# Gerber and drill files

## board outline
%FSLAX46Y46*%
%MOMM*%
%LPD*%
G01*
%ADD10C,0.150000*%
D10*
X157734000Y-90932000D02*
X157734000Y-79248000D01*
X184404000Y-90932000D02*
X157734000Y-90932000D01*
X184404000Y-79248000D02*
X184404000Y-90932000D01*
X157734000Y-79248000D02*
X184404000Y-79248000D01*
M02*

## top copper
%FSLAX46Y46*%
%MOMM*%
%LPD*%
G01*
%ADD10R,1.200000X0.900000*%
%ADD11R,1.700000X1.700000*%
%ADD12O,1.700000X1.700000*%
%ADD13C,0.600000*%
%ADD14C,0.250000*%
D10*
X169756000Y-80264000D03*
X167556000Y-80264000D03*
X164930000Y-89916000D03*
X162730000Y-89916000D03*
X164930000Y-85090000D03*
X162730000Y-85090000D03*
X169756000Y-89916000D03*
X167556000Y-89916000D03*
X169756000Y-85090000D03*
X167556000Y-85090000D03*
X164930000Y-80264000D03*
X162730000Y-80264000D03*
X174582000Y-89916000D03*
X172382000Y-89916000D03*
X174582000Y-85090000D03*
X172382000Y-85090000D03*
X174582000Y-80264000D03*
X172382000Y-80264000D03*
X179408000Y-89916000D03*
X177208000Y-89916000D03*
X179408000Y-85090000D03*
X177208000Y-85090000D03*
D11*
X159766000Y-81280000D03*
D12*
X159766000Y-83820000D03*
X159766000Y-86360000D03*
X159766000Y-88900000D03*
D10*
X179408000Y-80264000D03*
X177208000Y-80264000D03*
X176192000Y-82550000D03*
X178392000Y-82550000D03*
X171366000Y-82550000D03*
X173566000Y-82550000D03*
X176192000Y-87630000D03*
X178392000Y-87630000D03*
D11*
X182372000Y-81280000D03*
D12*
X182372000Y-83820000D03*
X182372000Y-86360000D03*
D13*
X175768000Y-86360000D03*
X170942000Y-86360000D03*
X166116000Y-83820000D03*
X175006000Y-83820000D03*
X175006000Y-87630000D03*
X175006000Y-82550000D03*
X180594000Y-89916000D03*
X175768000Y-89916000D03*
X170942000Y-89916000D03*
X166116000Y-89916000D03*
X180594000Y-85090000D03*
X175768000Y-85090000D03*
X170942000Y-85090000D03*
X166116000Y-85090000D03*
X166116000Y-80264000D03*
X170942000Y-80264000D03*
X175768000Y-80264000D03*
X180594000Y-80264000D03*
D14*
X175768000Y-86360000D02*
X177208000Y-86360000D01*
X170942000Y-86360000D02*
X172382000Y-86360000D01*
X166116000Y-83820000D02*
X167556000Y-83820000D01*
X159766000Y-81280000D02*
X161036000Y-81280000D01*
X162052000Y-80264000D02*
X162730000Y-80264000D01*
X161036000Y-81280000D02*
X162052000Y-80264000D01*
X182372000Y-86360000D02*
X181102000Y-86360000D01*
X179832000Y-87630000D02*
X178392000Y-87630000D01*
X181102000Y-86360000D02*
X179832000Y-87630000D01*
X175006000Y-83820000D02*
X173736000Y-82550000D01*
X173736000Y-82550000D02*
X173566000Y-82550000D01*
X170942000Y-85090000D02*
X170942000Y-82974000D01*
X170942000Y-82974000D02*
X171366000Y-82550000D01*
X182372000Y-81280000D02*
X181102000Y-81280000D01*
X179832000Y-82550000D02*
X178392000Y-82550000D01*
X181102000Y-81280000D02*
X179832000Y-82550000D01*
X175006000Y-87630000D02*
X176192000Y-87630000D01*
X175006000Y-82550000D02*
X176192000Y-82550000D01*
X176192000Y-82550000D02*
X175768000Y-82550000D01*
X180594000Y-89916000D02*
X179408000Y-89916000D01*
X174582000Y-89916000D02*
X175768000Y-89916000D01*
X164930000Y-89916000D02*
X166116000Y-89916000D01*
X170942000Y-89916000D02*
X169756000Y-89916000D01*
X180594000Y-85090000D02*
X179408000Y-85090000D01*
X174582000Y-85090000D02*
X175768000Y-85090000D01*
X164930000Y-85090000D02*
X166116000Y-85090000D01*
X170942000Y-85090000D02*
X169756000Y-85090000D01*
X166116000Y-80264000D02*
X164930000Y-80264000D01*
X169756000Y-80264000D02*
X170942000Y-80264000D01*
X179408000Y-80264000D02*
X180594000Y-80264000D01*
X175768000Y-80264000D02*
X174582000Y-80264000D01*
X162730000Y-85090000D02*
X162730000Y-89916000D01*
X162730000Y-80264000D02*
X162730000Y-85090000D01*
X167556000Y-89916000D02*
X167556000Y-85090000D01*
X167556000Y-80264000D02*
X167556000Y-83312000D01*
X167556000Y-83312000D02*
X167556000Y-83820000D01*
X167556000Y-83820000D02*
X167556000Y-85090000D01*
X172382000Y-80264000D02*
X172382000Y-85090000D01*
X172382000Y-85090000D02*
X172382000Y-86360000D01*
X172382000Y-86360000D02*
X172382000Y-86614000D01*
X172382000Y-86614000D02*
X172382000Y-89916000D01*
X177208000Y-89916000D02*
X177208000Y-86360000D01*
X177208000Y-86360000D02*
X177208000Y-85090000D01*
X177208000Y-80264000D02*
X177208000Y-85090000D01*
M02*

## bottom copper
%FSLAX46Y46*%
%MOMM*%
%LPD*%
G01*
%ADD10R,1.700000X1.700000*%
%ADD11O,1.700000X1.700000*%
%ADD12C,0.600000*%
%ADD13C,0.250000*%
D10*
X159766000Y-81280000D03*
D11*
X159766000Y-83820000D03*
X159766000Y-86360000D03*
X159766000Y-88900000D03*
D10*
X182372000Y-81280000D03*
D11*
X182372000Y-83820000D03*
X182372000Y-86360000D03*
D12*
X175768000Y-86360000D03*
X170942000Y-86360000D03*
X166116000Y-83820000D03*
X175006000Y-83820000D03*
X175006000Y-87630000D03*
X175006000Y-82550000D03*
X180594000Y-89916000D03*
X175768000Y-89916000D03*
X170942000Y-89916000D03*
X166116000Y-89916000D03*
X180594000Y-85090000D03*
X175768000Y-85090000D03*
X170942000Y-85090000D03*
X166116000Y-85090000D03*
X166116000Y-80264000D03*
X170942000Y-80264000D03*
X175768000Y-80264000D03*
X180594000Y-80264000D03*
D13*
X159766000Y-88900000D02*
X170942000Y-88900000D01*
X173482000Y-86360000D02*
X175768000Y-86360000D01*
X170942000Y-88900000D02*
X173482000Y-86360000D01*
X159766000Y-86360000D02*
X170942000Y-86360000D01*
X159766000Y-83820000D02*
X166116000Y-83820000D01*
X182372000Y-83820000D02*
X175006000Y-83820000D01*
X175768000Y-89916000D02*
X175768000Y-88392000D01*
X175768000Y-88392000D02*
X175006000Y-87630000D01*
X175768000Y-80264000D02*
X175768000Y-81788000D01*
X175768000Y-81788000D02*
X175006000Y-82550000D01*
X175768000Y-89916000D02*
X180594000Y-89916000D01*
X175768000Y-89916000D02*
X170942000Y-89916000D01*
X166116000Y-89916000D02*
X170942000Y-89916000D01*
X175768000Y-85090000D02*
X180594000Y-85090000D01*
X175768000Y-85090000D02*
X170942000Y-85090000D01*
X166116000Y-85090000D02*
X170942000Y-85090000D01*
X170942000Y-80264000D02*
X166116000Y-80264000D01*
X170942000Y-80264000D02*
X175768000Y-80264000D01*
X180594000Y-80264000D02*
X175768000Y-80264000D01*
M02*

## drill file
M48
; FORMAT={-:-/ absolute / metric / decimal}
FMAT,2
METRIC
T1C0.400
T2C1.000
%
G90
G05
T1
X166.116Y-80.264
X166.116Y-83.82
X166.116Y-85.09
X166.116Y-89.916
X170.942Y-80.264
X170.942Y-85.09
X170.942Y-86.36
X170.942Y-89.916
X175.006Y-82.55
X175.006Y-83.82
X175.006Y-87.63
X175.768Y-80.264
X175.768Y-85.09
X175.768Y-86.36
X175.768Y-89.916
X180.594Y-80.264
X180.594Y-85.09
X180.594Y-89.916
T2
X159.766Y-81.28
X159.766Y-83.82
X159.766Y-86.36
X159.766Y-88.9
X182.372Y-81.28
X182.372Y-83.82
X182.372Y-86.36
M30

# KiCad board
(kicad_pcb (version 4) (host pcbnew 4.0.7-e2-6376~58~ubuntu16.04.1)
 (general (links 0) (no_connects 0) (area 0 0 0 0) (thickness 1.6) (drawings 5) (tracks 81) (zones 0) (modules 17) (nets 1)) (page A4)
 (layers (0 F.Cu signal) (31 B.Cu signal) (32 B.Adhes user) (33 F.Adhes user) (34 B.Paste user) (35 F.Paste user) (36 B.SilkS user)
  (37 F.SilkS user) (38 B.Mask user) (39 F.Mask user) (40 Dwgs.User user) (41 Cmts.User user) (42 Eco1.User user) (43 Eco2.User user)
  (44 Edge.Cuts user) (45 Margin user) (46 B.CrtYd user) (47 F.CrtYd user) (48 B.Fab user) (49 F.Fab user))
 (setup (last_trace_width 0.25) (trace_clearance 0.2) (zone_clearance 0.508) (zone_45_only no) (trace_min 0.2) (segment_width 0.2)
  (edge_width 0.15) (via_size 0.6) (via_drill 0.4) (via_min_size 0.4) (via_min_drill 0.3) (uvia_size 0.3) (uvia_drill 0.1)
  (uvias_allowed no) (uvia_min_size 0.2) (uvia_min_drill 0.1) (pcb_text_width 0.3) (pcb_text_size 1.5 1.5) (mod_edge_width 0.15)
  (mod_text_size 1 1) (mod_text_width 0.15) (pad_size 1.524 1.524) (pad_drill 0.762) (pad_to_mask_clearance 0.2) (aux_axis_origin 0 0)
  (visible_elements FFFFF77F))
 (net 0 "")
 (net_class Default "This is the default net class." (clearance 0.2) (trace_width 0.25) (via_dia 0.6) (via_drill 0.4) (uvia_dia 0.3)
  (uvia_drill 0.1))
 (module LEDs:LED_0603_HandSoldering (layer F.Cu) (at 168.656 80.264 180)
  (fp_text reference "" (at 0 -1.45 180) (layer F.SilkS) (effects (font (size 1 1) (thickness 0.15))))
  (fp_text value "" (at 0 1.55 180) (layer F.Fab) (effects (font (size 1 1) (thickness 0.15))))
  (pad 1 smd rect (at -1.1 0 180) (size 1.2 0.9) (layers F.Cu F.Paste F.Mask))
  (pad 2 smd rect (at 1.1 0 180) (size 1.2 0.9) (layers F.Cu F.Paste F.Mask)))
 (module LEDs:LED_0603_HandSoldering (layer F.Cu) (at 163.83 89.916 180)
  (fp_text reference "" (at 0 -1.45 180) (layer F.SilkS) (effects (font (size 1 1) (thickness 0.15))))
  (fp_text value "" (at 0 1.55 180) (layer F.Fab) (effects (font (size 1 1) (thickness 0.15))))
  (pad 1 smd rect (at -1.1 0 180) (size 1.2 0.9) (layers F.Cu F.Paste F.Mask))
  (pad 2 smd rect (at 1.1 0 180) (size 1.2 0.9) (layers F.Cu F.Paste F.Mask)))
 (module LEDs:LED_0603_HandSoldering (layer F.Cu) (at 163.83 85.09 180)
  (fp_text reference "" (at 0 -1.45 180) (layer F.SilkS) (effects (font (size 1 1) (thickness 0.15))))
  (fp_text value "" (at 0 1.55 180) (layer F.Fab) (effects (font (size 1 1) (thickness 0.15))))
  (pad 1 smd rect (at -1.1 0 180) (size 1.2 0.9) (layers F.Cu F.Paste F.Mask))
  (pad 2 smd rect (at 1.1 0 180) (size 1.2 0.9) (layers F.Cu F.Paste F.Mask)))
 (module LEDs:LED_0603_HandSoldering (layer F.Cu) (at 168.656 89.916 180)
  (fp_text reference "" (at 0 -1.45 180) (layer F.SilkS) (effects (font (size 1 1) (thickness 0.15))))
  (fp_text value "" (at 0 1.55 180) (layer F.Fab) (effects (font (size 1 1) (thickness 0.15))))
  (pad 1 smd rect (at -1.1 0 180) (size 1.2 0.9) (layers F.Cu F.Paste F.Mask))
  (pad 2 smd rect (at 1.1 0 180) (size 1.2 0.9) (layers F.Cu F.Paste F.Mask)))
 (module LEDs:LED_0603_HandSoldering (layer F.Cu) (at 168.656 85.09 180)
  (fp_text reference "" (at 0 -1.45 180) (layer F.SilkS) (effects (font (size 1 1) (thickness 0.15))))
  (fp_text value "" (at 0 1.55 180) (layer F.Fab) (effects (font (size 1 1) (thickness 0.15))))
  (pad 1 smd rect (at -1.1 0 180) (size 1.2 0.9) (layers F.Cu F.Paste F.Mask))
  (pad 2 smd rect (at 1.1 0 180) (size 1.2 0.9) (layers F.Cu F.Paste F.Mask)))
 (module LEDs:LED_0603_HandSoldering (layer F.Cu) (at 163.83 80.264 180)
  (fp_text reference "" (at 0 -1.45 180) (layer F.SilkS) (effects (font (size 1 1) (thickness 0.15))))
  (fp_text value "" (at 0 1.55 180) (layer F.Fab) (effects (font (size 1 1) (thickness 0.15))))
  (pad 1 smd rect (at -1.1 0 180) (size 1.2 0.9) (layers F.Cu F.Paste F.Mask))
  (pad 2 smd rect (at 1.1 0 180) (size 1.2 0.9) (layers F.Cu F.Paste F.Mask)))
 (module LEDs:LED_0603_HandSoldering (layer F.Cu) (at 173.482 89.916 180)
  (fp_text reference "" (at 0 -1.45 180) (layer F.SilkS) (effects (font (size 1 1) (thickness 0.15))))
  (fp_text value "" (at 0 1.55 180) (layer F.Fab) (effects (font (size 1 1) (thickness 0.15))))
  (pad 1 smd rect (at -1.1 0 180) (size 1.2 0.9) (layers F.Cu F.Paste F.Mask))
  (pad 2 smd rect (at 1.1 0 180) (size 1.2 0.9) (layers F.Cu F.Paste F.Mask)))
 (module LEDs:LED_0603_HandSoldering (layer F.Cu) (at 173.482 85.09 180)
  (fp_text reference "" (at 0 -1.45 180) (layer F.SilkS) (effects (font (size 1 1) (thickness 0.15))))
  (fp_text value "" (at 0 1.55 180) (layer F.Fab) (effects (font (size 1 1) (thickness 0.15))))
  (pad 1 smd rect (at -1.1 0 180) (size 1.2 0.9) (layers F.Cu F.Paste F.Mask))
  (pad 2 smd rect (at 1.1 0 180) (size 1.2 0.9) (layers F.Cu F.Paste F.Mask)))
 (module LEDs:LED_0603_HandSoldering (layer F.Cu) (at 173.482 80.264 180)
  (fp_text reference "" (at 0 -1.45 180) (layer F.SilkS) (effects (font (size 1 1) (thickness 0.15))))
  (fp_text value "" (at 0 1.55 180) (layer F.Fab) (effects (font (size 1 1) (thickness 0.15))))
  (pad 1 smd rect (at -1.1 0 180) (size 1.2 0.9) (layers F.Cu F.Paste F.Mask))
  (pad 2 smd rect (at 1.1 0 180) (size 1.2 0.9) (layers F.Cu F.Paste F.Mask)))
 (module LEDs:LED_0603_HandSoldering (layer F.Cu) (at 178.308 89.916 180)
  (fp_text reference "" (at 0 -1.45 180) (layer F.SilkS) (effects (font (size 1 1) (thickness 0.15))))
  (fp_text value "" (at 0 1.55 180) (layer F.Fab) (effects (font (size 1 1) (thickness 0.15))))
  (pad 1 smd rect (at -1.1 0 180) (size 1.2 0.9) (layers F.Cu F.Paste F.Mask))
  (pad 2 smd rect (at 1.1 0 180) (size 1.2 0.9) (layers F.Cu F.Paste F.Mask)))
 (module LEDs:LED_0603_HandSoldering (layer F.Cu) (at 178.308 85.09 180)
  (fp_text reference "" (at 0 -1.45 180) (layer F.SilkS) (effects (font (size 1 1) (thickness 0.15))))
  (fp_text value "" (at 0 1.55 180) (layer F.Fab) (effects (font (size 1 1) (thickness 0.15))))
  (pad 1 smd rect (at -1.1 0 180) (size 1.2 0.9) (layers F.Cu F.Paste F.Mask))
  (pad 2 smd rect (at 1.1 0 180) (size 1.2 0.9) (layers F.Cu F.Paste F.Mask)))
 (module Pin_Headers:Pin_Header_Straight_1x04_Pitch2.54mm (layer F.Cu) (at 159.766 81.28)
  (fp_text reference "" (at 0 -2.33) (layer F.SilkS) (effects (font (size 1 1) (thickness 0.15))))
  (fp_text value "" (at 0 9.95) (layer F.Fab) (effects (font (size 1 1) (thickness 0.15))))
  (pad 1 thru_hole rect (at 0 0) (size 1.7 1.7) (drill 1) (layers *.Cu *.Mask))
  (pad 2 thru_hole oval (at 0 2.54) (size 1.7 1.7) (drill 1) (layers *.Cu *.Mask))
  (pad 3 thru_hole oval (at 0 5.08) (size 1.7 1.7) (drill 1) (layers *.Cu *.Mask))
  (pad 4 thru_hole oval (at 0 7.62) (size 1.7 1.7) (drill 1) (layers *.Cu *.Mask)))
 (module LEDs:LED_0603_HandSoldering (layer F.Cu) (at 178.308 80.264 180)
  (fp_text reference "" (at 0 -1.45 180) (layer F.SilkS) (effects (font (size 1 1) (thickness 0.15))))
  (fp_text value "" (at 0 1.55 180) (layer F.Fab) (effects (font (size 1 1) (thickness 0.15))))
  (pad 1 smd rect (at -1.1 0 180) (size 1.2 0.9) (layers F.Cu F.Paste F.Mask))
  (pad 2 smd rect (at 1.1 0 180) (size 1.2 0.9) (layers F.Cu F.Paste F.Mask)))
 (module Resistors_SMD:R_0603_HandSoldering (layer F.Cu) (at 177.292 82.55)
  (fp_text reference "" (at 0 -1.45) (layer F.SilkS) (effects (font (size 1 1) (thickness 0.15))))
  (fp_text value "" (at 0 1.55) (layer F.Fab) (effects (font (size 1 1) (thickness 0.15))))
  (pad 1 smd rect (at -1.1 0) (size 1.2 0.9) (layers F.Cu F.Paste F.Mask))
  (pad 2 smd rect (at 1.1 0) (size 1.2 0.9) (layers F.Cu F.Paste F.Mask)))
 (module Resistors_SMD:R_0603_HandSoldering (layer F.Cu) (at 172.466 82.55)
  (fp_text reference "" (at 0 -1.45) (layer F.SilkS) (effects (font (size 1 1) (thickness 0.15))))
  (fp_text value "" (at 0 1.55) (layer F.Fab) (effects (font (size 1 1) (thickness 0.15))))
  (pad 1 smd rect (at -1.1 0) (size 1.2 0.9) (layers F.Cu F.Paste F.Mask))
  (pad 2 smd rect (at 1.1 0) (size 1.2 0.9) (layers F.Cu F.Paste F.Mask)))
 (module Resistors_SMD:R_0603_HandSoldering (layer F.Cu) (at 177.292 87.63)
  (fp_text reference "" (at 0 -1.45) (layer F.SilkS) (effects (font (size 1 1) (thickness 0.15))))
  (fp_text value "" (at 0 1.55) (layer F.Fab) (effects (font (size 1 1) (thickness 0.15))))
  (pad 1 smd rect (at -1.1 0) (size 1.2 0.9) (layers F.Cu F.Paste F.Mask))
  (pad 2 smd rect (at 1.1 0) (size 1.2 0.9) (layers F.Cu F.Paste F.Mask)))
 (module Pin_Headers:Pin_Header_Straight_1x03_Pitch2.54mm (layer F.Cu) (at 182.372 81.28)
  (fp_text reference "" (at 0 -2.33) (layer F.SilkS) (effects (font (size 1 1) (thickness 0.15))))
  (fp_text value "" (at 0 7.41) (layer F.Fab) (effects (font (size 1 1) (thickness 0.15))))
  (pad 1 thru_hole rect (at 0 0) (size 1.7 1.7) (drill 1) (layers *.Cu *.Mask))
  (pad 2 thru_hole oval (at 0 2.54) (size 1.7 1.7) (drill 1) (layers *.Cu *.Mask))
  (pad 3 thru_hole oval (at 0 5.08) (size 1.7 1.7) (drill 1) (layers *.Cu *.Mask)))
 (gr_line (start 157.734 90.932) (end 157.734 79.248) (angle 90) (layer Edge.Cuts) (width 0.15))
 (gr_line (start 184.404 90.932) (end 157.734 90.932) (angle 90) (layer Edge.Cuts) (width 0.15))
 (gr_line (start 184.404 79.248) (end 184.404 90.932) (angle 90) (layer Edge.Cuts) (width 0.15))
 (gr_line (start 157.734 79.248) (end 184.404 79.248) (angle 90) (layer Edge.Cuts) (width 0.15))
 (segment (start 159.766 88.9) (end 170.942 88.9) (width 0.25) (layer B.Cu) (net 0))
 (segment (start 175.768 86.36) (end 177.208 86.36) (width 0.25) (layer F.Cu) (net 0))
 (via (at 175.768 86.36) (size 0.6) (drill 0.4) (layers F.Cu B.Cu) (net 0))
 (segment (start 173.482 86.36) (end 175.768 86.36) (width 0.25) (layer B.Cu) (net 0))
 (segment (start 170.942 88.9) (end 173.482 86.36) (width 0.25) (layer B.Cu) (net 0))
 (segment (start 159.766 86.36) (end 170.942 86.36) (width 0.25) (layer B.Cu) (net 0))
 (segment (start 170.942 86.36) (end 172.382 86.36) (width 0.25) (layer F.Cu) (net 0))
 (via (at 170.942 86.36) (size 0.6) (drill 0.4) (layers F.Cu B.Cu) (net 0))
 (segment (start 159.766 83.82) (end 166.116 83.82) (width 0.25) (layer B.Cu) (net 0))
 (segment (start 166.116 83.82) (end 167.556 83.82) (width 0.25) (layer F.Cu) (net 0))
 (via (at 166.116 83.82) (size 0.6) (drill 0.4) (layers F.Cu B.Cu) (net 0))
 (segment (start 159.766 81.28) (end 161.036 81.28) (width 0.25) (layer F.Cu) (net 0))
 (segment (start 162.052 80.264) (end 162.73 80.264) (width 0.25) (layer F.Cu) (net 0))
 (segment (start 161.036 81.28) (end 162.052 80.264) (width 0.25) (layer F.Cu) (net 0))
 (segment (start 182.372 86.36) (end 181.102 86.36) (width 0.25) (layer F.Cu) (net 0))
 (segment (start 179.832 87.63) (end 178.392 87.63) (width 0.25) (layer F.Cu) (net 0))
 (segment (start 181.102 86.36) (end 179.832 87.63) (width 0.25) (layer F.Cu) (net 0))
 (segment (start 182.372 83.82) (end 175.006 83.82) (width 0.25) (layer B.Cu) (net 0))
 (segment (start 175.006 83.82) (end 173.736 82.55) (width 0.25) (layer F.Cu) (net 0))
 (via (at 175.006 83.82) (size 0.6) (drill 0.4) (layers F.Cu B.Cu) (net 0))
 (segment (start 173.736 82.55) (end 173.566 82.55) (width 0.25) (layer F.Cu) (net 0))
 (segment (start 170.942 85.09) (end 170.942 82.974) (width 0.25) (layer F.Cu) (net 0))
 (segment (start 170.942 82.974) (end 171.366 82.55) (width 0.25) (layer F.Cu) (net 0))
 (segment (start 182.372 81.28) (end 181.102 81.28) (width 0.25) (layer F.Cu) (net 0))
 (segment (start 179.832 82.55) (end 178.392 82.55) (width 0.25) (layer F.Cu) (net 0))
 (segment (start 181.102 81.28) (end 179.832 82.55) (width 0.25) (layer F.Cu) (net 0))
 (segment (start 175.768 89.916) (end 175.768 88.392) (width 0.25) (layer B.Cu) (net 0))
 (segment (start 175.006 87.63) (end 176.192 87.63) (width 0.25) (layer F.Cu) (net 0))
 (via (at 175.006 87.63) (size 0.6) (drill 0.4) (layers F.Cu B.Cu) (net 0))
 (segment (start 175.768 88.392) (end 175.006 87.63) (width 0.25) (layer B.Cu) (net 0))
 (segment (start 175.768 80.264) (end 175.768 81.788) (width 0.25) (layer B.Cu) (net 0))
 (segment (start 175.006 82.55) (end 176.192 82.55) (width 0.25) (layer F.Cu) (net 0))
 (via (at 175.006 82.55) (size 0.6) (drill 0.4) (layers F.Cu B.Cu) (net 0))
 (segment (start 175.768 81.788) (end 175.006 82.55) (width 0.25) (layer B.Cu) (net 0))
 (segment (start 176.192 82.55) (end 175.768 82.55) (width 0.25) (layer F.Cu) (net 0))
 (segment (start 175.768 89.916) (end 180.594 89.916) (width 0.25) (layer B.Cu) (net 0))
 (segment (start 180.594 89.916) (end 179.408 89.916) (width 0.25) (layer F.Cu) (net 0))
 (via (at 180.594 89.916) (size 0.6) (drill 0.4) (layers F.Cu B.Cu) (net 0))
 (segment (start 174.582 89.916) (end 175.768 89.916) (width 0.25) (layer F.Cu) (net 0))
 (segment (start 175.768 89.916) (end 170.942 89.916) (width 0.25) (layer B.Cu) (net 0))
 (via (at 175.768 89.916) (size 0.6) (drill 0.4) (layers F.Cu B.Cu) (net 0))
 (segment (start 164.93 89.916) (end 166.116 89.916) (width 0.25) (layer F.Cu) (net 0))
 (segment (start 170.942 89.916) (end 169.756 89.916) (width 0.25) (layer F.Cu) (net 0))
 (via (at 170.942 89.916) (size 0.6) (drill 0.4) (layers F.Cu B.Cu) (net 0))
 (segment (start 166.116 89.916) (end 170.942 89.916) (width 0.25) (layer B.Cu) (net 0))
 (via (at 166.116 89.916) (size 0.6) (drill 0.4) (layers F.Cu B.Cu) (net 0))
 (segment (start 175.768 85.09) (end 180.594 85.09) (width 0.25) (layer B.Cu) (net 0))
 (segment (start 180.594 85.09) (end 179.408 85.09) (width 0.25) (layer F.Cu) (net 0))
 (via (at 180.594 85.09) (size 0.6) (drill 0.4) (layers F.Cu B.Cu) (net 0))
 (segment (start 174.582 85.09) (end 175.768 85.09) (width 0.25) (layer F.Cu) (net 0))
 (segment (start 175.768 85.09) (end 170.942 85.09) (width 0.25) (layer B.Cu) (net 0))
 (via (at 175.768 85.09) (size 0.6) (drill 0.4) (layers F.Cu B.Cu) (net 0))
 (segment (start 164.93 85.09) (end 166.116 85.09) (width 0.25) (layer F.Cu) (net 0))
 (segment (start 170.942 85.09) (end 169.756 85.09) (width 0.25) (layer F.Cu) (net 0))
 (via (at 170.942 85.09) (size 0.6) (drill 0.4) (layers F.Cu B.Cu) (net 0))
 (segment (start 166.116 85.09) (end 170.942 85.09) (width 0.25) (layer B.Cu) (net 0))
 (via (at 166.116 85.09) (size 0.6) (drill 0.4) (layers F.Cu B.Cu) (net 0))
 (segment (start 170.942 80.264) (end 166.116 80.264) (width 0.25) (layer B.Cu) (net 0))
 (segment (start 166.116 80.264) (end 164.93 80.264) (width 0.25) (layer F.Cu) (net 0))
 (via (at 166.116 80.264) (size 0.6) (drill 0.4) (layers F.Cu B.Cu) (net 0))
 (segment (start 169.756 80.264) (end 170.942 80.264) (width 0.25) (layer F.Cu) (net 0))
 (segment (start 170.942 80.264) (end 175.768 80.264) (width 0.25) (layer B.Cu) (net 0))
 (via (at 170.942 80.264) (size 0.6) (drill 0.4) (layers F.Cu B.Cu) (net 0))
 (segment (start 179.408 80.264) (end 180.594 80.264) (width 0.25) (layer F.Cu) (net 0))
 (segment (start 175.768 80.264) (end 174.582 80.264) (width 0.25) (layer F.Cu) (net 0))
 (via (at 175.768 80.264) (size 0.6) (drill 0.4) (layers F.Cu B.Cu) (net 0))
 (segment (start 180.594 80.264) (end 175.768 80.264) (width 0.25) (layer B.Cu) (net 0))
 (via (at 180.594 80.264) (size 0.6) (drill 0.4) (layers F.Cu B.Cu) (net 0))
 (segment (start 162.73 85.09) (end 162.73 89.916) (width 0.25) (layer F.Cu) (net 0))
 (segment (start 162.73 80.264) (end 162.73 85.09) (width 0.25) (layer F.Cu) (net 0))
 (segment (start 167.556 89.916) (end 167.556 85.09) (width 0.25) (layer F.Cu) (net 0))
 (segment (start 167.556 80.264) (end 167.556 83.312) (width 0.25) (layer F.Cu) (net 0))
 (segment (start 167.556 83.312) (end 167.556 83.82) (width 0.25) (layer F.Cu) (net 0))
 (segment (start 167.556 83.82) (end 167.556 85.09) (width 0.25) (layer F.Cu) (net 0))
 (segment (start 172.382 80.264) (end 172.382 85.09) (width 0.25) (layer F.Cu) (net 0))
 (segment (start 172.382 85.09) (end 172.382 86.36) (width 0.25) (layer F.Cu) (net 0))
 (segment (start 172.382 86.36) (end 172.382 86.614) (width 0.25) (layer F.Cu) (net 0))
 (segment (start 172.382 86.614) (end 172.382 89.916) (width 0.25) (layer F.Cu) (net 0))
 (segment (start 177.208 89.916) (end 177.208 86.36) (width 0.25) (layer F.Cu) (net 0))
 (segment (start 177.208 86.36) (end 177.208 85.09) (width 0.25) (layer F.Cu) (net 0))
 (segment (start 177.208 80.264) (end 177.208 85.09) (width 0.25) (layer F.Cu) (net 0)))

